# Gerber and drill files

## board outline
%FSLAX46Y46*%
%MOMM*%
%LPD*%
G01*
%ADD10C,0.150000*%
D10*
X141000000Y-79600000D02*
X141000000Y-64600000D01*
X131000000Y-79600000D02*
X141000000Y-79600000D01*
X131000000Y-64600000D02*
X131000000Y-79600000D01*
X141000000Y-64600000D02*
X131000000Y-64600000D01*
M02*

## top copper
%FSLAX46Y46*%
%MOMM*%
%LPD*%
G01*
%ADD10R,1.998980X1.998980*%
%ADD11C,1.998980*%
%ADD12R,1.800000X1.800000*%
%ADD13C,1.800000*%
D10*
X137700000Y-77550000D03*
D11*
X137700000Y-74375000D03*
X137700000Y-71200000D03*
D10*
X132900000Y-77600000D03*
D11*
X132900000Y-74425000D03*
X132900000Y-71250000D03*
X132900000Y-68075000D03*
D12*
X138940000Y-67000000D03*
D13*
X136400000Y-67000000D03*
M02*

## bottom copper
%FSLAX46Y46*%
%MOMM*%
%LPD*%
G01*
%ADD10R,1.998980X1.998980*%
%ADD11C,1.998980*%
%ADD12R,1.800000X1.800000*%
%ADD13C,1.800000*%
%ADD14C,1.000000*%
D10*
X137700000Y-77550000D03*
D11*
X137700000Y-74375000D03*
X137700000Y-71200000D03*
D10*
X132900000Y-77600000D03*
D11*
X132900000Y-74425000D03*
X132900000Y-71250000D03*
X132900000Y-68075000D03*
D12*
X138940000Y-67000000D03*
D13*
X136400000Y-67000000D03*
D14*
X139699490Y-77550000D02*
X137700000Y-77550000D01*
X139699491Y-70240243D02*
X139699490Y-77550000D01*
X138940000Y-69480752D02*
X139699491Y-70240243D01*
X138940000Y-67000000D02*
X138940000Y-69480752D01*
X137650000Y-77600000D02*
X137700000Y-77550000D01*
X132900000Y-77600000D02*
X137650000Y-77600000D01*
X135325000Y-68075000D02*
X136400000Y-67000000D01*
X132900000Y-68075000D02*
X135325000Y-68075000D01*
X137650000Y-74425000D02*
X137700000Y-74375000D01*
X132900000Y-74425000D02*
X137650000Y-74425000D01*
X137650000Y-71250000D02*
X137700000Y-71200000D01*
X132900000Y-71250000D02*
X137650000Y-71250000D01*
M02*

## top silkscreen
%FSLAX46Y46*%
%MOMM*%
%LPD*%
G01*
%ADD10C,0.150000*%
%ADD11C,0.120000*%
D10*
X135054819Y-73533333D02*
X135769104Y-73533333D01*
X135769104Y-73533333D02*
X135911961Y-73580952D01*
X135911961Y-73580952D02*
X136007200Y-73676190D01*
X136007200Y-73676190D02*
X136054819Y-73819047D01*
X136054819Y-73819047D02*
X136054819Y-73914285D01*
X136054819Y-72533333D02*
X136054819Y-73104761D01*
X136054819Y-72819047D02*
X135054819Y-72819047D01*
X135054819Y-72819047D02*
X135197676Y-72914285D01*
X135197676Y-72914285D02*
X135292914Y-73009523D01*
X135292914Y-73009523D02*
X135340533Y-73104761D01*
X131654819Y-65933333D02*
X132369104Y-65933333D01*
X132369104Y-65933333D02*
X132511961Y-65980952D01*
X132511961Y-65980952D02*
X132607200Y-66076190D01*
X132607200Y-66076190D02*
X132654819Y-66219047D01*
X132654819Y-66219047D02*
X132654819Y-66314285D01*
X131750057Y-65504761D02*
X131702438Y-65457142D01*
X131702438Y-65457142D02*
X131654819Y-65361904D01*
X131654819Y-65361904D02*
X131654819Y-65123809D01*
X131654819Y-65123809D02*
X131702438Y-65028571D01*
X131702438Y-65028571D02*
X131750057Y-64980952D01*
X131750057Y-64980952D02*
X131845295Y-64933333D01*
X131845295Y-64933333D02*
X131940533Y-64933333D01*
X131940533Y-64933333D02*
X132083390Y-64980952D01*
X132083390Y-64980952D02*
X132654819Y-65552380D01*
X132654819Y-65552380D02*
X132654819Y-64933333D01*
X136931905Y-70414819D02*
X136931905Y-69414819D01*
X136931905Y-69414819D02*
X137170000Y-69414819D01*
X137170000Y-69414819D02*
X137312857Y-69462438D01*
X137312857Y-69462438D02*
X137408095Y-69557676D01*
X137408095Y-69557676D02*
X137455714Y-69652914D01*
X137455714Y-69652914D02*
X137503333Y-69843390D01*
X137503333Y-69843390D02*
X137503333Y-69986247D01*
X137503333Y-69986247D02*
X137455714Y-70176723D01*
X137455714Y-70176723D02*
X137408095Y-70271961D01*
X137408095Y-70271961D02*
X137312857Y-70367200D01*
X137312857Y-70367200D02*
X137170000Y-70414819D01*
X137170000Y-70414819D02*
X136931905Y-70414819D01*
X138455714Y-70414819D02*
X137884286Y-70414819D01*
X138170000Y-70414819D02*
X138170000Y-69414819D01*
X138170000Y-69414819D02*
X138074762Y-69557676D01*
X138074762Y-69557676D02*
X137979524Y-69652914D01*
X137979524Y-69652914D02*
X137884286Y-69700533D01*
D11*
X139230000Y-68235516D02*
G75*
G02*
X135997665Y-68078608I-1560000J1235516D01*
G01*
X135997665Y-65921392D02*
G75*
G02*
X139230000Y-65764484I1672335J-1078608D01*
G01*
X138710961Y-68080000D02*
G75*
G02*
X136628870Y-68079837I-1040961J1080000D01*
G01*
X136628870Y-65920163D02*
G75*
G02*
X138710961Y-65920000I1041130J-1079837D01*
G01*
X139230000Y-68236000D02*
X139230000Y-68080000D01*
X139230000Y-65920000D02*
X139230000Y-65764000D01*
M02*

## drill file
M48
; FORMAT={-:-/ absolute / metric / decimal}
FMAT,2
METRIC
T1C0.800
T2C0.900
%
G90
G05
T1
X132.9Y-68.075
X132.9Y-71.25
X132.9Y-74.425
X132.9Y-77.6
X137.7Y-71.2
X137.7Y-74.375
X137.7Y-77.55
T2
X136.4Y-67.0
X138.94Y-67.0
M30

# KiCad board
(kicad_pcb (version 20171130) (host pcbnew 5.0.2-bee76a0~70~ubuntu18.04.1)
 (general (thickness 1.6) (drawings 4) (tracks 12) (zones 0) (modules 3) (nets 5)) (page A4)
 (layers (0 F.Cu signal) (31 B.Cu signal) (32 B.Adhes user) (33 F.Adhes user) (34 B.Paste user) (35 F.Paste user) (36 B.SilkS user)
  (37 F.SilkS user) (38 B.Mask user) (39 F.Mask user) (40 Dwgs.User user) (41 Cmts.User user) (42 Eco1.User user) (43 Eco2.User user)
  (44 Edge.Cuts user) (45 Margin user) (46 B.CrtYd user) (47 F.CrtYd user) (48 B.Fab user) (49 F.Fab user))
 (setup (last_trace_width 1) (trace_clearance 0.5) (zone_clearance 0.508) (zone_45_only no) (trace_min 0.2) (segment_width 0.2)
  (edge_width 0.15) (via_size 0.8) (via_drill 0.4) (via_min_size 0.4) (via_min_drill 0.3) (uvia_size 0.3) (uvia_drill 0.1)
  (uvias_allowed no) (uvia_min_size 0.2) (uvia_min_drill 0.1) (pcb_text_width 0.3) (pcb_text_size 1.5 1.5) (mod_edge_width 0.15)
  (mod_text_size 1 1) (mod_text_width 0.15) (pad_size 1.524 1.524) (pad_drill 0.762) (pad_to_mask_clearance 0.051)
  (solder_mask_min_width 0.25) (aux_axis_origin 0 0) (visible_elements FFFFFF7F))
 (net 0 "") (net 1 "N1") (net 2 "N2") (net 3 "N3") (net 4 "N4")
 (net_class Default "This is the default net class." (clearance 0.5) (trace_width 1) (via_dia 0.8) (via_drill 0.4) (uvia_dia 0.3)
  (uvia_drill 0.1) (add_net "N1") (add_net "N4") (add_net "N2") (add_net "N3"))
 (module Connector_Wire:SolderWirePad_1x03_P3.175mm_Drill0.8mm (layer F.Cu) (at 137.7 77.55 90)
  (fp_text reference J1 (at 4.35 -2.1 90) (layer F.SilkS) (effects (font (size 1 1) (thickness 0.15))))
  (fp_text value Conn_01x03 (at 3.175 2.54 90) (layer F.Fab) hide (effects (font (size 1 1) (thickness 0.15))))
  (pad 1 thru_hole rect (at 0 0 90) (size 1.99898 1.99898) (drill 0.8001) (layers *.Cu *.Mask) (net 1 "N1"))
  (pad 2 thru_hole circle (at 3.175 0 90) (size 1.99898 1.99898) (drill 0.8001) (layers *.Cu *.Mask) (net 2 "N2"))
  (pad 3 thru_hole circle (at 6.35 0 90) (size 1.99898 1.99898) (drill 0.8001) (layers *.Cu *.Mask) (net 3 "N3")))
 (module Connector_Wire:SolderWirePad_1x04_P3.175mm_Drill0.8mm (layer F.Cu) (at 132.9 77.6 90)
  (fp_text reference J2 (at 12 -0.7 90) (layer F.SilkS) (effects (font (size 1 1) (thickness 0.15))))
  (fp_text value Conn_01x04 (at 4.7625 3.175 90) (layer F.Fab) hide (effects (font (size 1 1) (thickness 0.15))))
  (pad 1 thru_hole rect (at 0 0 90) (size 1.99898 1.99898) (drill 0.8001) (layers *.Cu *.Mask) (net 1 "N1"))
  (pad 2 thru_hole circle (at 3.175 0 90) (size 1.99898 1.99898) (drill 0.8001) (layers *.Cu *.Mask) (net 2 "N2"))
  (pad 3 thru_hole circle (at 6.35 0 90) (size 1.99898 1.99898) (drill 0.8001) (layers *.Cu *.Mask) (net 3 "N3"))
  (pad 4 thru_hole circle (at 9.525 0 90) (size 1.99898 1.99898) (drill 0.8001) (layers *.Cu *.Mask) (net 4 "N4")))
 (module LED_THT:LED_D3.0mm (layer F.Cu) (at 138.94 67 180)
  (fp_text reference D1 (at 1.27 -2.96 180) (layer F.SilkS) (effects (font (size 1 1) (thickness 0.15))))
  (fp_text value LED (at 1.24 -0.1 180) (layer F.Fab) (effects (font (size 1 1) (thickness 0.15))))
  (fp_arc (start 1.27 0) (end -0.29 -1.235516) (angle 108.8) (layer F.SilkS) (width 0.12))
  (fp_arc (start 1.27 0) (end -0.29 1.235516) (angle -108.8) (layer F.SilkS) (width 0.12))
  (fp_arc (start 1.27 0) (end 0.229039 -1.08) (angle 87.9) (layer F.SilkS) (width 0.12))
  (fp_arc (start 1.27 0) (end 0.229039 1.08) (angle -87.9) (layer F.SilkS) (width 0.12))
  (fp_line (start -0.29 -1.236) (end -0.29 -1.08) (layer F.SilkS) (width 0.12))
  (fp_line (start -0.29 1.08) (end -0.29 1.236) (layer F.SilkS) (width 0.12))
  (pad 1 thru_hole rect (at 0 0 180) (size 1.8 1.8) (drill 0.9) (layers *.Cu *.Mask) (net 1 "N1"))
  (pad 2 thru_hole circle (at 2.54 0 180) (size 1.8 1.8) (drill 0.9) (layers *.Cu *.Mask) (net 4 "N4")))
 (gr_line (start 141 79.6) (end 141 64.6) (layer Edge.Cuts) (width 0.15))
 (gr_line (start 131 79.6) (end 141 79.6) (layer Edge.Cuts) (width 0.15))
 (gr_line (start 131 64.6) (end 131 79.6) (layer Edge.Cuts) (width 0.15))
 (gr_line (start 141 64.6) (end 131 64.6) (layer Edge.Cuts) (width 0.15))
 (segment (start 139.69949 77.55) (end 137.7 77.55) (width 1) (layer B.Cu) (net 1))
 (segment (start 139.699491 70.240243) (end 139.69949 77.55) (width 1) (layer B.Cu) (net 1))
 (segment (start 138.94 69.480752) (end 139.699491 70.240243) (width 1) (layer B.Cu) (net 1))
 (segment (start 138.94 67) (end 138.94 69.480752) (width 1) (layer B.Cu) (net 1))
 (segment (start 137.65 77.6) (end 137.7 77.55) (width 1) (layer B.Cu) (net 1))
 (segment (start 132.9 77.6) (end 137.65 77.6) (width 1) (layer B.Cu) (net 1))
 (segment (start 135.325 68.075) (end 136.4 67) (width 1) (layer B.Cu) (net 4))
 (segment (start 132.9 68.075) (end 135.325 68.075) (width 1) (layer B.Cu) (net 4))
 (segment (start 137.65 74.425) (end 137.7 74.375) (width 1) (layer B.Cu) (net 2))
 (segment (start 132.9 74.425) (end 137.65 74.425) (width 1) (layer B.Cu) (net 2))
 (segment (start 137.65 71.25) (end 137.7 71.2) (width 1) (layer B.Cu) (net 3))
 (segment (start 132.9 71.25) (end 137.65 71.25) (width 1) (layer B.Cu) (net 3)))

